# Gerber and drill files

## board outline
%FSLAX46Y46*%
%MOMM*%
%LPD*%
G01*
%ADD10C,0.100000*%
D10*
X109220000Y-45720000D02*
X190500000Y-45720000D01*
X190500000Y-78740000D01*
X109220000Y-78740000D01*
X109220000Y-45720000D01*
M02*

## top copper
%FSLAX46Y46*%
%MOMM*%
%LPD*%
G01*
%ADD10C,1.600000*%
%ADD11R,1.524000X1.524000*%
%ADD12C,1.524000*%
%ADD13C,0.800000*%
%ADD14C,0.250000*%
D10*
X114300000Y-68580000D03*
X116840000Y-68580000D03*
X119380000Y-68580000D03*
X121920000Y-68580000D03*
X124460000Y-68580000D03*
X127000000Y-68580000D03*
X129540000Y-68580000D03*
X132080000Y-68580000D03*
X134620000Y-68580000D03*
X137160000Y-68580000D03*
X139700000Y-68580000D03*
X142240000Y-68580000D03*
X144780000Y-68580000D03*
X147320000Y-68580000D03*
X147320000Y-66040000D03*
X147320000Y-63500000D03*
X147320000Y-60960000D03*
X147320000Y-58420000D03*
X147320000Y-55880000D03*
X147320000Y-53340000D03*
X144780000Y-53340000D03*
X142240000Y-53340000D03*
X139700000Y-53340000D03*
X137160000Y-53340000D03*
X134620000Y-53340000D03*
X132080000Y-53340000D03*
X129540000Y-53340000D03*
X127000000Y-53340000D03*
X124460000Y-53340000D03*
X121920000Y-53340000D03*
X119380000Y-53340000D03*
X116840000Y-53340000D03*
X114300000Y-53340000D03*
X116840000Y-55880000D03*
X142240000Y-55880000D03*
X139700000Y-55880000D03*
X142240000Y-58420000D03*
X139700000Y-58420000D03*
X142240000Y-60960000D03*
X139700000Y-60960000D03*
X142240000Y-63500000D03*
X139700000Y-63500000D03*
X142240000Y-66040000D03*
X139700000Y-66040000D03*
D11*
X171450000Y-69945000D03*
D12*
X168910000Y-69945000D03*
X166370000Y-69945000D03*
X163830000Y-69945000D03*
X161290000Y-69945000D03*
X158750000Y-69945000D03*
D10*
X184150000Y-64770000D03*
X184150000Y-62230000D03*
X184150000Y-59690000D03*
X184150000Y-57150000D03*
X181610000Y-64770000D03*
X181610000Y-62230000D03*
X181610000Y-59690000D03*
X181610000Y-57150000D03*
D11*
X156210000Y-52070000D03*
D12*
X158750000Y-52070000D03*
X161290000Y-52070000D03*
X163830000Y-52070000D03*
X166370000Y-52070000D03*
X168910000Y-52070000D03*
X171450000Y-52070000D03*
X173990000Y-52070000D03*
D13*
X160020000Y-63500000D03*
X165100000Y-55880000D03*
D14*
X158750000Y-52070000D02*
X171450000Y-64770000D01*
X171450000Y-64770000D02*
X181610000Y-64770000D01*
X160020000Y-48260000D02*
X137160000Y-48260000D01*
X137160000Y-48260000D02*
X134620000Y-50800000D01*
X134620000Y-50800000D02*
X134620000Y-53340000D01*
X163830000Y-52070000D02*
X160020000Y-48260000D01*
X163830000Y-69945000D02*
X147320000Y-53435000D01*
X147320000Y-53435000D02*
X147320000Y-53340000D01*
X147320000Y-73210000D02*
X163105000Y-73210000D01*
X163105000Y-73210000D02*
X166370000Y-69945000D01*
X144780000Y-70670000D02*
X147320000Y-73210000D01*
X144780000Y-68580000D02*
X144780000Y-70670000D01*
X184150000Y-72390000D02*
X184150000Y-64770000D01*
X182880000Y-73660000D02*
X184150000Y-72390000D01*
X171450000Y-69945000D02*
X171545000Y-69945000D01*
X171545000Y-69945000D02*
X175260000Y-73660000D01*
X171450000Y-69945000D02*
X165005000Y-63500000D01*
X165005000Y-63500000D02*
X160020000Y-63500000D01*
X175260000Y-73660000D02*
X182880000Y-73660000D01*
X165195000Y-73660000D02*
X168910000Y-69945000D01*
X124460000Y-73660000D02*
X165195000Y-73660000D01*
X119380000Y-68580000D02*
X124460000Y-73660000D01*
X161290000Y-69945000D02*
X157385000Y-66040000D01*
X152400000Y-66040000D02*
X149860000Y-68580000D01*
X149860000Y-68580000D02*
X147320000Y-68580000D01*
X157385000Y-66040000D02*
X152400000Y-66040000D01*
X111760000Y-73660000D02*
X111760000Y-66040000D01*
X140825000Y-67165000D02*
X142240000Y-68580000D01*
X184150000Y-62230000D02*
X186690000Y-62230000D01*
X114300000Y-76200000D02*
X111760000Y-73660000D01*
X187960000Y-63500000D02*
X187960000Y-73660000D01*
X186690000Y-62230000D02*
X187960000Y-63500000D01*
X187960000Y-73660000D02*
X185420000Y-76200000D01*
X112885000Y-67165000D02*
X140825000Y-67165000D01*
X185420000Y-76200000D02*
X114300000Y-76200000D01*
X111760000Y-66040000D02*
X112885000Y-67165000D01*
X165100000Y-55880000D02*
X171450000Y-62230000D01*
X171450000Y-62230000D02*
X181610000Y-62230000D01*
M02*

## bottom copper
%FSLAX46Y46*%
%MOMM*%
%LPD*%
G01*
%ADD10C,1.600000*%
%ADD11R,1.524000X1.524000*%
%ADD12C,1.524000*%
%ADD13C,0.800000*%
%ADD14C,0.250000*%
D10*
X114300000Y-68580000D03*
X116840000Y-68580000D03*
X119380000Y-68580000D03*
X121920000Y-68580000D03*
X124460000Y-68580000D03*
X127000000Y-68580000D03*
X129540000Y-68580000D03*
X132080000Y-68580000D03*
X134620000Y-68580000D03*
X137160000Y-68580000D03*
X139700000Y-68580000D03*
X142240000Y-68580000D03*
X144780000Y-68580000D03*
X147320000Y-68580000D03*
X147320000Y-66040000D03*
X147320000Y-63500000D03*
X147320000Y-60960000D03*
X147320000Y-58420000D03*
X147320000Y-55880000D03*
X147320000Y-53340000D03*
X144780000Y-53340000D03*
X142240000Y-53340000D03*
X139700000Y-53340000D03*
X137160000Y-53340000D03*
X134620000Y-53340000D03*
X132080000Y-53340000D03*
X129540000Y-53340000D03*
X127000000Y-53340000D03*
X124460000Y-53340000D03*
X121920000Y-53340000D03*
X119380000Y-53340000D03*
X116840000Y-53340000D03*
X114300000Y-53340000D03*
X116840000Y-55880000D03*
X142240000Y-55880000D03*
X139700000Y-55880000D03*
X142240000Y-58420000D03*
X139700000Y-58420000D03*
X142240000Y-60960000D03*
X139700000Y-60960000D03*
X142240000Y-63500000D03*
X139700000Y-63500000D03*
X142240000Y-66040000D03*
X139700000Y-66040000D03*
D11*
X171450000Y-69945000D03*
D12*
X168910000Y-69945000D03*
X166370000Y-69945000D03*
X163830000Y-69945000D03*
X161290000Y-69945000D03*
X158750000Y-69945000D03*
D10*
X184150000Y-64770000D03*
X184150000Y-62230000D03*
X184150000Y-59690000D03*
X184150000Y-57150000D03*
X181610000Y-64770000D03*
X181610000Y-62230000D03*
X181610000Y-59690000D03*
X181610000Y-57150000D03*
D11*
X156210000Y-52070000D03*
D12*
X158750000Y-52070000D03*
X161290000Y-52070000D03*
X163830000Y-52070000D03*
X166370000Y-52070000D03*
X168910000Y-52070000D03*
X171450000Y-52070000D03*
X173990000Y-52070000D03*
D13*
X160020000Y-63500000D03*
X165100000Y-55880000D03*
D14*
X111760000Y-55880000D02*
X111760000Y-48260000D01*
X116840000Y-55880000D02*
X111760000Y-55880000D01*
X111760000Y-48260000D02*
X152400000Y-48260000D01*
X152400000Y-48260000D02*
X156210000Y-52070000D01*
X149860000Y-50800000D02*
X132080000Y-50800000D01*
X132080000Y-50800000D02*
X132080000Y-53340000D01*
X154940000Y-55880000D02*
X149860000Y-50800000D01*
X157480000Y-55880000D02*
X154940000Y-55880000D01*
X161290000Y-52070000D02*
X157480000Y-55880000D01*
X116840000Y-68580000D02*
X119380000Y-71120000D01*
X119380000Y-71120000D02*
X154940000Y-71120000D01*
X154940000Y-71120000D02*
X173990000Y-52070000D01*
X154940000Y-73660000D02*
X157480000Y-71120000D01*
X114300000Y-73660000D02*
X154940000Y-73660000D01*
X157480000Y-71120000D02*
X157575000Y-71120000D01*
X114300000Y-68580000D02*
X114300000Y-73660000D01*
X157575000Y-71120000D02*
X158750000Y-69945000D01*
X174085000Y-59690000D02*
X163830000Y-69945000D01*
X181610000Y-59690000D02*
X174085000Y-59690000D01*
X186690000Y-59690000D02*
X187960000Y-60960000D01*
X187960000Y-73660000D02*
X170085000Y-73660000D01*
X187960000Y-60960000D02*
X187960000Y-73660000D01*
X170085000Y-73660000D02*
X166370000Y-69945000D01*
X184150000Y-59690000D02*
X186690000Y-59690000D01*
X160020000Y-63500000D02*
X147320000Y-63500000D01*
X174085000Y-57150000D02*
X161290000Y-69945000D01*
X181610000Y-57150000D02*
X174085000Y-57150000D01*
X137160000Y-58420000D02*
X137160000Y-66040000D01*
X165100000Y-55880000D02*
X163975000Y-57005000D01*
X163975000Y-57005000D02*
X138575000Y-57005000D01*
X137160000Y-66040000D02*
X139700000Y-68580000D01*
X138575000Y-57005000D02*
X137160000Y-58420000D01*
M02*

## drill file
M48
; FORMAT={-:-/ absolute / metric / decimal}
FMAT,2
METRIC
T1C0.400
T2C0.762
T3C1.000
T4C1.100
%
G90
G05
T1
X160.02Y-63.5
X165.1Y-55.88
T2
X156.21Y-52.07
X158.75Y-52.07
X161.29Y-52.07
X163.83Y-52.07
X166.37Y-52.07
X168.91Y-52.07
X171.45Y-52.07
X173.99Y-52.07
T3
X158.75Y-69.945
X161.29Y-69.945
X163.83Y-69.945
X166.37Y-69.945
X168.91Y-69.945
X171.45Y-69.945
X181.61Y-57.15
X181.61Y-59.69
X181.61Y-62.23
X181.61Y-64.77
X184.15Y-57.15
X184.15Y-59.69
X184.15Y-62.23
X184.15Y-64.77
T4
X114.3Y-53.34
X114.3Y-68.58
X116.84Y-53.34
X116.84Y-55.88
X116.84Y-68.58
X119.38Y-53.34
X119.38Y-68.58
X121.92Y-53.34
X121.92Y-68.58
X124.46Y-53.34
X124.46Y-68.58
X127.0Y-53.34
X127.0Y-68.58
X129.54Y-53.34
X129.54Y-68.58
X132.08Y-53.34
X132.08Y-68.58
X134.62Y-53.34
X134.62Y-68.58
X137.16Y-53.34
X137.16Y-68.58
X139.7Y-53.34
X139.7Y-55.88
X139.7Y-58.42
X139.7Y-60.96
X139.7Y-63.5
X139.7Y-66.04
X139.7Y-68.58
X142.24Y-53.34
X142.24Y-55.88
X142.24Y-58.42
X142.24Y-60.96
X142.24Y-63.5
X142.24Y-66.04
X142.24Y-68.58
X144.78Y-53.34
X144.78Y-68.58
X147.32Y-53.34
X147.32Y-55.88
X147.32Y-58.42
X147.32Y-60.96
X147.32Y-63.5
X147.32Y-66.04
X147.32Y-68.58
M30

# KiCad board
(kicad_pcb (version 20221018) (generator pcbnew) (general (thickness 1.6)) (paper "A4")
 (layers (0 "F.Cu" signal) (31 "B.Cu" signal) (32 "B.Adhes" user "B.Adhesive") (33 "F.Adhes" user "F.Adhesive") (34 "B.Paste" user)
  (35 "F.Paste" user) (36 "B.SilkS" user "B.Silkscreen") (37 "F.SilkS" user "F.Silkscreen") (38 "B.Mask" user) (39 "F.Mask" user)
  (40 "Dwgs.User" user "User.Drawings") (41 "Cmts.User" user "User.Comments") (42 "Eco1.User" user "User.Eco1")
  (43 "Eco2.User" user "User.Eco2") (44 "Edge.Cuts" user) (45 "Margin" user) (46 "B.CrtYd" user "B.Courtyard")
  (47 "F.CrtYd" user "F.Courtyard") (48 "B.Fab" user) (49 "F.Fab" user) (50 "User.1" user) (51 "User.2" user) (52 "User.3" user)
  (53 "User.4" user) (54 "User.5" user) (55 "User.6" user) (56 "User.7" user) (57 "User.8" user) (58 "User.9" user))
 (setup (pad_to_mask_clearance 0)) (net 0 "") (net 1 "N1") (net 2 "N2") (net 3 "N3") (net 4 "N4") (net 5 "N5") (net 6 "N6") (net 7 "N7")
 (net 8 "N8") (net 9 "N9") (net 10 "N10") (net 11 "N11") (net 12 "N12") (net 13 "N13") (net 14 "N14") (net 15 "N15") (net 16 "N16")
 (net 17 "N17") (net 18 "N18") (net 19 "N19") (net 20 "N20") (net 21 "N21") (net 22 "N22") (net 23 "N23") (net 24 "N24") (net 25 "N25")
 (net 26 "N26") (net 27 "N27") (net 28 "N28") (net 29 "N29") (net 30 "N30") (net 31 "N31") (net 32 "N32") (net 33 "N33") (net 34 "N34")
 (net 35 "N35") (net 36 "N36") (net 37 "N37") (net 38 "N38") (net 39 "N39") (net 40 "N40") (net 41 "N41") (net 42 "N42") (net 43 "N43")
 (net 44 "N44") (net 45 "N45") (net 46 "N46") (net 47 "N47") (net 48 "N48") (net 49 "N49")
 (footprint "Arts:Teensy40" (layer "F.Cu") (at 130.81 60.96)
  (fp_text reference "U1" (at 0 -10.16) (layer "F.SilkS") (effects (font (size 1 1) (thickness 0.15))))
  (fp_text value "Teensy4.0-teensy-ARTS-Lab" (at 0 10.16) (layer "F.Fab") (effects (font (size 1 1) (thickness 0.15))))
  (pad "1" thru_hole circle (at -16.51 7.62) (size 1.6 1.6) (drill 1.1) (layers "*.Cu" "*.Mask") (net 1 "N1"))
  (pad "2" thru_hole circle (at -13.97 7.62) (size 1.6 1.6) (drill 1.1) (layers "*.Cu" "*.Mask") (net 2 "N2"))
  (pad "3" thru_hole circle (at -11.43 7.62) (size 1.6 1.6) (drill 1.1) (layers "*.Cu" "*.Mask") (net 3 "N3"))
  (pad "4" thru_hole circle (at -8.89 7.62) (size 1.6 1.6) (drill 1.1) (layers "*.Cu" "*.Mask") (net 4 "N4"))
  (pad "5" thru_hole circle (at -6.35 7.62) (size 1.6 1.6) (drill 1.1) (layers "*.Cu" "*.Mask") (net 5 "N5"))
  (pad "6" thru_hole circle (at -3.81 7.62) (size 1.6 1.6) (drill 1.1) (layers "*.Cu" "*.Mask") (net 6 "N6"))
  (pad "7" thru_hole circle (at -1.27 7.62) (size 1.6 1.6) (drill 1.1) (layers "*.Cu" "*.Mask") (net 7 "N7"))
  (pad "8" thru_hole circle (at 1.27 7.62) (size 1.6 1.6) (drill 1.1) (layers "*.Cu" "*.Mask") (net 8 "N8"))
  (pad "9" thru_hole circle (at 3.81 7.62) (size 1.6 1.6) (drill 1.1) (layers "*.Cu" "*.Mask") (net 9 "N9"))
  (pad "10" thru_hole circle (at 6.35 7.62) (size 1.6 1.6) (drill 1.1) (layers "*.Cu" "*.Mask") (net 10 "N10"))
  (pad "11" thru_hole circle (at 8.89 7.62) (size 1.6 1.6) (drill 1.1) (layers "*.Cu" "*.Mask") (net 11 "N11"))
  (pad "12" thru_hole circle (at 11.43 7.62) (size 1.6 1.6) (drill 1.1) (layers "*.Cu" "*.Mask") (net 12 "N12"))
  (pad "13" thru_hole circle (at 13.97 7.62) (size 1.6 1.6) (drill 1.1) (layers "*.Cu" "*.Mask") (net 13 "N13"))
  (pad "14" thru_hole circle (at 16.51 7.62) (size 1.6 1.6) (drill 1.1) (layers "*.Cu" "*.Mask") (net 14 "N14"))
  (pad "15" thru_hole circle (at 16.51 5.08) (size 1.6 1.6) (drill 1.1) (layers "*.Cu" "*.Mask") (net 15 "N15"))
  (pad "16" thru_hole circle (at 16.51 2.54) (size 1.6 1.6) (drill 1.1) (layers "*.Cu" "*.Mask") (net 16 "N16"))
  (pad "17" thru_hole circle (at 16.51 0) (size 1.6 1.6) (drill 1.1) (layers "*.Cu" "*.Mask") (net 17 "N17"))
  (pad "18" thru_hole circle (at 16.51 -2.54) (size 1.6 1.6) (drill 1.1) (layers "*.Cu" "*.Mask") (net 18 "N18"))
  (pad "19" thru_hole circle (at 16.51 -5.08) (size 1.6 1.6) (drill 1.1) (layers "*.Cu" "*.Mask") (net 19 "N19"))
  (pad "20" thru_hole circle (at 16.51 -7.62) (size 1.6 1.6) (drill 1.1) (layers "*.Cu" "*.Mask") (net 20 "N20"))
  (pad "21" thru_hole circle (at 13.97 -7.62) (size 1.6 1.6) (drill 1.1) (layers "*.Cu" "*.Mask") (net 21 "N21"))
  (pad "22" thru_hole circle (at 11.43 -7.62) (size 1.6 1.6) (drill 1.1) (layers "*.Cu" "*.Mask") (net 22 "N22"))
  (pad "23" thru_hole circle (at 8.89 -7.62) (size 1.6 1.6) (drill 1.1) (layers "*.Cu" "*.Mask") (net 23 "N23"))
  (pad "24" thru_hole circle (at 6.35 -7.62) (size 1.6 1.6) (drill 1.1) (layers "*.Cu" "*.Mask") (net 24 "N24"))
  (pad "25" thru_hole circle (at 3.81 -7.62) (size 1.6 1.6) (drill 1.1) (layers "*.Cu" "*.Mask") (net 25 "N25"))
  (pad "26" thru_hole circle (at 1.27 -7.62) (size 1.6 1.6) (drill 1.1) (layers "*.Cu" "*.Mask") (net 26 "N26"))
  (pad "27" thru_hole circle (at -1.27 -7.62) (size 1.6 1.6) (drill 1.1) (layers "*.Cu" "*.Mask") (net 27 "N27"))
  (pad "28" thru_hole circle (at -3.81 -7.62) (size 1.6 1.6) (drill 1.1) (layers "*.Cu" "*.Mask") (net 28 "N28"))
  (pad "29" thru_hole circle (at -6.35 -7.62) (size 1.6 1.6) (drill 1.1) (layers "*.Cu" "*.Mask") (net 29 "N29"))
  (pad "30" thru_hole circle (at -8.89 -7.62) (size 1.6 1.6) (drill 1.1) (layers "*.Cu" "*.Mask") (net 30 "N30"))
  (pad "31" thru_hole circle (at -11.43 -7.62) (size 1.6 1.6) (drill 1.1) (layers "*.Cu" "*.Mask") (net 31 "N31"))
  (pad "32" thru_hole circle (at -13.97 -7.62) (size 1.6 1.6) (drill 1.1) (layers "*.Cu" "*.Mask") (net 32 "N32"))
  (pad "33" thru_hole circle (at -16.51 -7.62) (size 1.6 1.6) (drill 1.1) (layers "*.Cu" "*.Mask") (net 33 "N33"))
  (pad "34" thru_hole circle (at -13.97 -5.08) (size 1.6 1.6) (drill 1.1) (layers "*.Cu" "*.Mask") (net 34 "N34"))
  (pad "35" thru_hole circle (at 11.43 -5.08) (size 1.6 1.6) (drill 1.1) (layers "*.Cu" "*.Mask") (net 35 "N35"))
  (pad "36" thru_hole circle (at 8.89 -5.08) (size 1.6 1.6) (drill 1.1) (layers "*.Cu" "*.Mask") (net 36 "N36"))
  (pad "37" thru_hole circle (at 11.43 -2.54) (size 1.6 1.6) (drill 1.1) (layers "*.Cu" "*.Mask") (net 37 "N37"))
  (pad "38" thru_hole circle (at 8.89 -2.54) (size 1.6 1.6) (drill 1.1) (layers "*.Cu" "*.Mask") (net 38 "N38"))
  (pad "39" thru_hole circle (at 11.43 0) (size 1.6 1.6) (drill 1.1) (layers "*.Cu" "*.Mask") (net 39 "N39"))
  (pad "40" thru_hole circle (at 8.89 0) (size 1.6 1.6) (drill 1.1) (layers "*.Cu" "*.Mask") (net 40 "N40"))
  (pad "41" thru_hole circle (at 11.43 2.54) (size 1.6 1.6) (drill 1.1) (layers "*.Cu" "*.Mask") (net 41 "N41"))
  (pad "42" thru_hole circle (at 8.89 2.54) (size 1.6 1.6) (drill 1.1) (layers "*.Cu" "*.Mask") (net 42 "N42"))
  (pad "43" thru_hole circle (at 11.43 5.08) (size 1.6 1.6) (drill 1.1) (layers "*.Cu" "*.Mask") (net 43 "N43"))
  (pad "44" thru_hole circle (at 8.89 5.08) (size 1.6 1.6) (drill 1.1) (layers "*.Cu" "*.Mask") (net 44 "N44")))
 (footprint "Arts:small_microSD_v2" (layer "F.Cu") (at 164.465 66.77)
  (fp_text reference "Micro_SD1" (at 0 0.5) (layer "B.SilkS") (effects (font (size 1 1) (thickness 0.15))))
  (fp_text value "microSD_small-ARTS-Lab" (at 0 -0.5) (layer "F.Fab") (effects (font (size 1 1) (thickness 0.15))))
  (pad "1" thru_hole rect (at 6.985 3.175) (size 1.524 1.524) (drill 1) (layers "*.Cu" "*.Mask") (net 16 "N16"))
  (pad "2" thru_hole circle (at 4.445 3.175) (size 1.524 1.524) (drill 1) (layers "*.Cu" "*.Mask") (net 3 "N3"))
  (pad "3" thru_hole circle (at 1.905 3.175) (size 1.524 1.524) (drill 1) (layers "*.Cu" "*.Mask") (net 13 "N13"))
  (pad "4" thru_hole circle (at -0.635 3.175) (size 1.524 1.524) (drill 1) (layers "*.Cu" "*.Mask") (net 20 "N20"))
  (pad "5" thru_hole circle (at -3.175 3.175) (size 1.524 1.524) (drill 1) (layers "*.Cu" "*.Mask") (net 14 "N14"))
  (pad "6" thru_hole circle (at -5.715 3.175) (size 1.524 1.524) (drill 1) (layers "*.Cu" "*.Mask") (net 1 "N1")))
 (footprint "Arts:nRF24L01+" (layer "F.Cu") (at 193.04 58.42 -90)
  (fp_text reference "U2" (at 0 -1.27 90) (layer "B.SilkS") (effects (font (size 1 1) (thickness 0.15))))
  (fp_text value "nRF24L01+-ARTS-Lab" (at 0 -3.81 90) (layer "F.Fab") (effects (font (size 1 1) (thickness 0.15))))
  (pad "1" thru_hole circle (at 6.35 8.89 270) (size 1.6 1.6) (drill 1) (layers "*.Cu" "*.Mask") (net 16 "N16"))
  (pad "2" thru_hole circle (at 3.81 8.89 270) (size 1.6 1.6) (drill 1) (layers "*.Cu" "*.Mask") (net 12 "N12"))
  (pad "3" thru_hole circle (at 1.27 8.89 270) (size 1.6 1.6) (drill 1) (layers "*.Cu" "*.Mask") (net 13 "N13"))
  (pad "4" thru_hole circle (at -1.27 8.89 270) (size 1.6 1.6) (drill 1) (layers "*.Cu" "*.Mask") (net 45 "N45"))
  (pad "5" thru_hole circle (at 6.35 11.43 270) (size 1.6 1.6) (drill 1) (layers "*.Cu" "*.Mask") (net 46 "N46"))
  (pad "6" thru_hole circle (at 3.81 11.43 270) (size 1.6 1.6) (drill 1) (layers "*.Cu" "*.Mask") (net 11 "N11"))
  (pad "7" thru_hole circle (at 1.27 11.43 270) (size 1.6 1.6) (drill 1) (layers "*.Cu" "*.Mask") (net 20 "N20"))
  (pad "8" thru_hole circle (at -1.27 11.43 270) (size 1.6 1.6) (drill 1) (layers "*.Cu" "*.Mask") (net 14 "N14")))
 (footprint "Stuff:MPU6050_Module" (layer "F.Cu") (at 156.21 52.07 90)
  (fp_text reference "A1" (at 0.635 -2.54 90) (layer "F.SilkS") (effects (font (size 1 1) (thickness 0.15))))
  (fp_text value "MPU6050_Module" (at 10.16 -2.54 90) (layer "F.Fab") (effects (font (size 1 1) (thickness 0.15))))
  (pad "1" thru_hole rect (at 0 0 90) (size 1.524 1.524) (drill 0.762) (layers "*.Cu" "*.Mask") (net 34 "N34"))
  (pad "2" thru_hole circle (at 0 2.54 90) (size 1.524 1.524) (drill 0.762) (layers "*.Cu" "*.Mask") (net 46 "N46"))
  (pad "3" thru_hole circle (at 0 5.08 90) (size 1.524 1.524) (drill 0.762) (layers "*.Cu" "*.Mask") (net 26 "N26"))
  (pad "4" thru_hole circle (at 0 7.62 90) (size 1.524 1.524) (drill 0.762) (layers "*.Cu" "*.Mask") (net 25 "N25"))
  (pad "5" thru_hole circle (at 0 10.16 90) (size 1.524 1.524) (drill 0.762) (layers "*.Cu" "*.Mask") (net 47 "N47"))
  (pad "6" thru_hole circle (at 0 12.7 90) (size 1.524 1.524) (drill 0.762) (layers "*.Cu" "*.Mask") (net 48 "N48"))
  (pad "7" thru_hole circle (at 0 15.24 90) (size 1.524 1.524) (drill 0.762) (layers "*.Cu" "*.Mask") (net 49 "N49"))
  (pad "8" thru_hole circle (at 0 17.78 90) (size 1.524 1.524) (drill 0.762) (layers "*.Cu" "*.Mask") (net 2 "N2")))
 (gr_rect (start 109.22 45.72) (end 190.5 78.74) (stroke (width 0.1) (type default)) (fill none) (layer "Edge.Cuts"))
 (segment (start 111.76 55.88) (end 111.76 48.26) (width 0.25) (layer "B.Cu") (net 34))
 (segment (start 116.84 55.88) (end 111.76 55.88) (width 0.25) (layer "B.Cu") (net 34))
 (segment (start 111.76 48.26) (end 152.4 48.26) (width 0.25) (layer "B.Cu") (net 34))
 (segment (start 152.4 48.26) (end 156.21 52.07) (width 0.25) (layer "B.Cu") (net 34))
 (segment (start 158.75 52.07) (end 171.45 64.77) (width 0.25) (layer "F.Cu") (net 46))
 (segment (start 171.45 64.77) (end 181.61 64.77) (width 0.25) (layer "F.Cu") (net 46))
 (segment (start 149.86 50.8) (end 132.08 50.8) (width 0.25) (layer "B.Cu") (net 26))
 (segment (start 132.08 50.8) (end 132.08 53.34) (width 0.25) (layer "B.Cu") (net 26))
 (segment (start 154.94 55.88) (end 149.86 50.8) (width 0.25) (layer "B.Cu") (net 26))
 (segment (start 157.48 55.88) (end 154.94 55.88) (width 0.25) (layer "B.Cu") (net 26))
 (segment (start 161.29 52.07) (end 157.48 55.88) (width 0.25) (layer "B.Cu") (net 26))
 (segment (start 160.02 48.26) (end 137.16 48.26) (width 0.25) (layer "F.Cu") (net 25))
 (segment (start 137.16 48.26) (end 134.62 50.8) (width 0.25) (layer "F.Cu") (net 25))
 (segment (start 134.62 50.8) (end 134.62 53.34) (width 0.25) (layer "F.Cu") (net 25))
 (segment (start 163.83 52.07) (end 160.02 48.26) (width 0.25) (layer "F.Cu") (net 25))
 (segment (start 116.84 68.58) (end 119.38 71.12) (width 0.25) (layer "B.Cu") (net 2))
 (segment (start 119.38 71.12) (end 154.94 71.12) (width 0.25) (layer "B.Cu") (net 2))
 (segment (start 154.94 71.12) (end 173.99 52.07) (width 0.25) (layer "B.Cu") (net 2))
 (segment (start 154.94 73.66) (end 157.48 71.12) (width 0.25) (layer "B.Cu") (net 1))
 (segment (start 114.3 73.66) (end 154.94 73.66) (width 0.25) (layer "B.Cu") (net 1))
 (segment (start 157.48 71.12) (end 157.575 71.12) (width 0.25) (layer "B.Cu") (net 1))
 (segment (start 114.3 68.58) (end 114.3 73.66) (width 0.25) (layer "B.Cu") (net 1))
 (segment (start 157.575 71.12) (end 158.75 69.945) (width 0.25) (layer "B.Cu") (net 1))
 (segment (start 163.83 69.945) (end 147.32 53.435) (width 0.25) (layer "F.Cu") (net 20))
 (segment (start 147.32 53.435) (end 147.32 53.34) (width 0.25) (layer "F.Cu") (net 20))
 (segment (start 174.085 59.69) (end 163.83 69.945) (width 0.25) (layer "B.Cu") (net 20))
 (segment (start 181.61 59.69) (end 174.085 59.69) (width 0.25) (layer "B.Cu") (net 20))
 (segment (start 147.32 73.21) (end 163.105 73.21) (width 0.25) (layer "F.Cu") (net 13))
 (segment (start 163.105 73.21) (end 166.37 69.945) (width 0.25) (layer "F.Cu") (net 13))
 (segment (start 144.78 70.67) (end 147.32 73.21) (width 0.25) (layer "F.Cu") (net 13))
 (segment (start 144.78 68.58) (end 144.78 70.67) (width 0.25) (layer "F.Cu") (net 13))
 (segment (start 186.69 59.69) (end 187.96 60.96) (width 0.25) (layer "B.Cu") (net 13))
 (segment (start 187.96 73.66) (end 170.085 73.66) (width 0.25) (layer "B.Cu") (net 13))
 (segment (start 187.96 60.96) (end 187.96 73.66) (width 0.25) (layer "B.Cu") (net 13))
 (segment (start 170.085 73.66) (end 166.37 69.945) (width 0.25) (layer "B.Cu") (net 13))
 (segment (start 184.15 59.69) (end 186.69 59.69) (width 0.25) (layer "B.Cu") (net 13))
 (segment (start 184.15 72.39) (end 184.15 64.77) (width 0.25) (layer "F.Cu") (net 16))
 (segment (start 182.88 73.66) (end 184.15 72.39) (width 0.25) (layer "F.Cu") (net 16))
 (segment (start 171.45 69.945) (end 171.545 69.945) (width 0.25) (layer "F.Cu") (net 16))
 (segment (start 171.545 69.945) (end 175.26 73.66) (width 0.25) (layer "F.Cu") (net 16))
 (segment (start 171.45 69.945) (end 165.005 63.5) (width 0.25) (layer "F.Cu") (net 16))
 (segment (start 165.005 63.5) (end 160.02 63.5) (width 0.25) (layer "F.Cu") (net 16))
 (segment (start 175.26 73.66) (end 182.88 73.66) (width 0.25) (layer "F.Cu") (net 16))
 (via (at 160.02 63.5) (size 0.8) (drill 0.4) (layers "F.Cu" "B.Cu") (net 16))
 (segment (start 160.02 63.5) (end 147.32 63.5) (width 0.25) (layer "B.Cu") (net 16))
 (segment (start 165.195 73.66) (end 168.91 69.945) (width 0.25) (layer "F.Cu") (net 3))
 (segment (start 124.46 73.66) (end 165.195 73.66) (width 0.25) (layer "F.Cu") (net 3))
 (segment (start 119.38 68.58) (end 124.46 73.66) (width 0.25) (layer "F.Cu") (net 3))
 (segment (start 161.29 69.945) (end 157.385 66.04) (width 0.25) (layer "F.Cu") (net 14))
 (segment (start 152.4 66.04) (end 149.86 68.58) (width 0.25) (layer "F.Cu") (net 14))
 (segment (start 149.86 68.58) (end 147.32 68.58) (width 0.25) (layer "F.Cu") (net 14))
 (segment (start 157.385 66.04) (end 152.4 66.04) (width 0.25) (layer "F.Cu") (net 14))
 (segment (start 174.085 57.15) (end 161.29 69.945) (width 0.25) (layer "B.Cu") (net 14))
 (segment (start 181.61 57.15) (end 174.085 57.15) (width 0.25) (layer "B.Cu") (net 14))
 (segment (start 111.76 73.66) (end 111.76 66.04) (width 0.25) (layer "F.Cu") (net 12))
 (segment (start 140.825 67.165) (end 142.24 68.58) (width 0.25) (layer "F.Cu") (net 12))
 (segment (start 184.15 62.23) (end 186.69 62.23) (width 0.25) (layer "F.Cu") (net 12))
 (segment (start 114.3 76.2) (end 111.76 73.66) (width 0.25) (layer "F.Cu") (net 12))
 (segment (start 187.96 63.5) (end 187.96 73.66) (width 0.25) (layer "F.Cu") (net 12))
 (segment (start 186.69 62.23) (end 187.96 63.5) (width 0.25) (layer "F.Cu") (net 12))
 (segment (start 187.96 73.66) (end 185.42 76.2) (width 0.25) (layer "F.Cu") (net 12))
 (segment (start 112.885 67.165) (end 140.825 67.165) (width 0.25) (layer "F.Cu") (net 12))
 (segment (start 185.42 76.2) (end 114.3 76.2) (width 0.25) (layer "F.Cu") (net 12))
 (segment (start 111.76 66.04) (end 112.885 67.165) (width 0.25) (layer "F.Cu") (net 12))
 (segment (start 165.1 55.88) (end 171.45 62.23) (width 0.25) (layer "F.Cu") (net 11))
 (segment (start 171.45 62.23) (end 181.61 62.23) (width 0.25) (layer "F.Cu") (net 11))
 (via (at 165.1 55.88) (size 0.8) (drill 0.4) (layers "F.Cu" "B.Cu") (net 11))
 (segment (start 137.16 58.42) (end 137.16 66.04) (width 0.25) (layer "B.Cu") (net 11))
 (segment (start 165.1 55.88) (end 163.975 57.005) (width 0.25) (layer "B.Cu") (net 11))
 (segment (start 163.975 57.005) (end 138.575 57.005) (width 0.25) (layer "B.Cu") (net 11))
 (segment (start 137.16 66.04) (end 139.7 68.58) (width 0.25) (layer "B.Cu") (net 11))
 (segment (start 138.575 57.005) (end 137.16 58.42) (width 0.25) (layer "B.Cu") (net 11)))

